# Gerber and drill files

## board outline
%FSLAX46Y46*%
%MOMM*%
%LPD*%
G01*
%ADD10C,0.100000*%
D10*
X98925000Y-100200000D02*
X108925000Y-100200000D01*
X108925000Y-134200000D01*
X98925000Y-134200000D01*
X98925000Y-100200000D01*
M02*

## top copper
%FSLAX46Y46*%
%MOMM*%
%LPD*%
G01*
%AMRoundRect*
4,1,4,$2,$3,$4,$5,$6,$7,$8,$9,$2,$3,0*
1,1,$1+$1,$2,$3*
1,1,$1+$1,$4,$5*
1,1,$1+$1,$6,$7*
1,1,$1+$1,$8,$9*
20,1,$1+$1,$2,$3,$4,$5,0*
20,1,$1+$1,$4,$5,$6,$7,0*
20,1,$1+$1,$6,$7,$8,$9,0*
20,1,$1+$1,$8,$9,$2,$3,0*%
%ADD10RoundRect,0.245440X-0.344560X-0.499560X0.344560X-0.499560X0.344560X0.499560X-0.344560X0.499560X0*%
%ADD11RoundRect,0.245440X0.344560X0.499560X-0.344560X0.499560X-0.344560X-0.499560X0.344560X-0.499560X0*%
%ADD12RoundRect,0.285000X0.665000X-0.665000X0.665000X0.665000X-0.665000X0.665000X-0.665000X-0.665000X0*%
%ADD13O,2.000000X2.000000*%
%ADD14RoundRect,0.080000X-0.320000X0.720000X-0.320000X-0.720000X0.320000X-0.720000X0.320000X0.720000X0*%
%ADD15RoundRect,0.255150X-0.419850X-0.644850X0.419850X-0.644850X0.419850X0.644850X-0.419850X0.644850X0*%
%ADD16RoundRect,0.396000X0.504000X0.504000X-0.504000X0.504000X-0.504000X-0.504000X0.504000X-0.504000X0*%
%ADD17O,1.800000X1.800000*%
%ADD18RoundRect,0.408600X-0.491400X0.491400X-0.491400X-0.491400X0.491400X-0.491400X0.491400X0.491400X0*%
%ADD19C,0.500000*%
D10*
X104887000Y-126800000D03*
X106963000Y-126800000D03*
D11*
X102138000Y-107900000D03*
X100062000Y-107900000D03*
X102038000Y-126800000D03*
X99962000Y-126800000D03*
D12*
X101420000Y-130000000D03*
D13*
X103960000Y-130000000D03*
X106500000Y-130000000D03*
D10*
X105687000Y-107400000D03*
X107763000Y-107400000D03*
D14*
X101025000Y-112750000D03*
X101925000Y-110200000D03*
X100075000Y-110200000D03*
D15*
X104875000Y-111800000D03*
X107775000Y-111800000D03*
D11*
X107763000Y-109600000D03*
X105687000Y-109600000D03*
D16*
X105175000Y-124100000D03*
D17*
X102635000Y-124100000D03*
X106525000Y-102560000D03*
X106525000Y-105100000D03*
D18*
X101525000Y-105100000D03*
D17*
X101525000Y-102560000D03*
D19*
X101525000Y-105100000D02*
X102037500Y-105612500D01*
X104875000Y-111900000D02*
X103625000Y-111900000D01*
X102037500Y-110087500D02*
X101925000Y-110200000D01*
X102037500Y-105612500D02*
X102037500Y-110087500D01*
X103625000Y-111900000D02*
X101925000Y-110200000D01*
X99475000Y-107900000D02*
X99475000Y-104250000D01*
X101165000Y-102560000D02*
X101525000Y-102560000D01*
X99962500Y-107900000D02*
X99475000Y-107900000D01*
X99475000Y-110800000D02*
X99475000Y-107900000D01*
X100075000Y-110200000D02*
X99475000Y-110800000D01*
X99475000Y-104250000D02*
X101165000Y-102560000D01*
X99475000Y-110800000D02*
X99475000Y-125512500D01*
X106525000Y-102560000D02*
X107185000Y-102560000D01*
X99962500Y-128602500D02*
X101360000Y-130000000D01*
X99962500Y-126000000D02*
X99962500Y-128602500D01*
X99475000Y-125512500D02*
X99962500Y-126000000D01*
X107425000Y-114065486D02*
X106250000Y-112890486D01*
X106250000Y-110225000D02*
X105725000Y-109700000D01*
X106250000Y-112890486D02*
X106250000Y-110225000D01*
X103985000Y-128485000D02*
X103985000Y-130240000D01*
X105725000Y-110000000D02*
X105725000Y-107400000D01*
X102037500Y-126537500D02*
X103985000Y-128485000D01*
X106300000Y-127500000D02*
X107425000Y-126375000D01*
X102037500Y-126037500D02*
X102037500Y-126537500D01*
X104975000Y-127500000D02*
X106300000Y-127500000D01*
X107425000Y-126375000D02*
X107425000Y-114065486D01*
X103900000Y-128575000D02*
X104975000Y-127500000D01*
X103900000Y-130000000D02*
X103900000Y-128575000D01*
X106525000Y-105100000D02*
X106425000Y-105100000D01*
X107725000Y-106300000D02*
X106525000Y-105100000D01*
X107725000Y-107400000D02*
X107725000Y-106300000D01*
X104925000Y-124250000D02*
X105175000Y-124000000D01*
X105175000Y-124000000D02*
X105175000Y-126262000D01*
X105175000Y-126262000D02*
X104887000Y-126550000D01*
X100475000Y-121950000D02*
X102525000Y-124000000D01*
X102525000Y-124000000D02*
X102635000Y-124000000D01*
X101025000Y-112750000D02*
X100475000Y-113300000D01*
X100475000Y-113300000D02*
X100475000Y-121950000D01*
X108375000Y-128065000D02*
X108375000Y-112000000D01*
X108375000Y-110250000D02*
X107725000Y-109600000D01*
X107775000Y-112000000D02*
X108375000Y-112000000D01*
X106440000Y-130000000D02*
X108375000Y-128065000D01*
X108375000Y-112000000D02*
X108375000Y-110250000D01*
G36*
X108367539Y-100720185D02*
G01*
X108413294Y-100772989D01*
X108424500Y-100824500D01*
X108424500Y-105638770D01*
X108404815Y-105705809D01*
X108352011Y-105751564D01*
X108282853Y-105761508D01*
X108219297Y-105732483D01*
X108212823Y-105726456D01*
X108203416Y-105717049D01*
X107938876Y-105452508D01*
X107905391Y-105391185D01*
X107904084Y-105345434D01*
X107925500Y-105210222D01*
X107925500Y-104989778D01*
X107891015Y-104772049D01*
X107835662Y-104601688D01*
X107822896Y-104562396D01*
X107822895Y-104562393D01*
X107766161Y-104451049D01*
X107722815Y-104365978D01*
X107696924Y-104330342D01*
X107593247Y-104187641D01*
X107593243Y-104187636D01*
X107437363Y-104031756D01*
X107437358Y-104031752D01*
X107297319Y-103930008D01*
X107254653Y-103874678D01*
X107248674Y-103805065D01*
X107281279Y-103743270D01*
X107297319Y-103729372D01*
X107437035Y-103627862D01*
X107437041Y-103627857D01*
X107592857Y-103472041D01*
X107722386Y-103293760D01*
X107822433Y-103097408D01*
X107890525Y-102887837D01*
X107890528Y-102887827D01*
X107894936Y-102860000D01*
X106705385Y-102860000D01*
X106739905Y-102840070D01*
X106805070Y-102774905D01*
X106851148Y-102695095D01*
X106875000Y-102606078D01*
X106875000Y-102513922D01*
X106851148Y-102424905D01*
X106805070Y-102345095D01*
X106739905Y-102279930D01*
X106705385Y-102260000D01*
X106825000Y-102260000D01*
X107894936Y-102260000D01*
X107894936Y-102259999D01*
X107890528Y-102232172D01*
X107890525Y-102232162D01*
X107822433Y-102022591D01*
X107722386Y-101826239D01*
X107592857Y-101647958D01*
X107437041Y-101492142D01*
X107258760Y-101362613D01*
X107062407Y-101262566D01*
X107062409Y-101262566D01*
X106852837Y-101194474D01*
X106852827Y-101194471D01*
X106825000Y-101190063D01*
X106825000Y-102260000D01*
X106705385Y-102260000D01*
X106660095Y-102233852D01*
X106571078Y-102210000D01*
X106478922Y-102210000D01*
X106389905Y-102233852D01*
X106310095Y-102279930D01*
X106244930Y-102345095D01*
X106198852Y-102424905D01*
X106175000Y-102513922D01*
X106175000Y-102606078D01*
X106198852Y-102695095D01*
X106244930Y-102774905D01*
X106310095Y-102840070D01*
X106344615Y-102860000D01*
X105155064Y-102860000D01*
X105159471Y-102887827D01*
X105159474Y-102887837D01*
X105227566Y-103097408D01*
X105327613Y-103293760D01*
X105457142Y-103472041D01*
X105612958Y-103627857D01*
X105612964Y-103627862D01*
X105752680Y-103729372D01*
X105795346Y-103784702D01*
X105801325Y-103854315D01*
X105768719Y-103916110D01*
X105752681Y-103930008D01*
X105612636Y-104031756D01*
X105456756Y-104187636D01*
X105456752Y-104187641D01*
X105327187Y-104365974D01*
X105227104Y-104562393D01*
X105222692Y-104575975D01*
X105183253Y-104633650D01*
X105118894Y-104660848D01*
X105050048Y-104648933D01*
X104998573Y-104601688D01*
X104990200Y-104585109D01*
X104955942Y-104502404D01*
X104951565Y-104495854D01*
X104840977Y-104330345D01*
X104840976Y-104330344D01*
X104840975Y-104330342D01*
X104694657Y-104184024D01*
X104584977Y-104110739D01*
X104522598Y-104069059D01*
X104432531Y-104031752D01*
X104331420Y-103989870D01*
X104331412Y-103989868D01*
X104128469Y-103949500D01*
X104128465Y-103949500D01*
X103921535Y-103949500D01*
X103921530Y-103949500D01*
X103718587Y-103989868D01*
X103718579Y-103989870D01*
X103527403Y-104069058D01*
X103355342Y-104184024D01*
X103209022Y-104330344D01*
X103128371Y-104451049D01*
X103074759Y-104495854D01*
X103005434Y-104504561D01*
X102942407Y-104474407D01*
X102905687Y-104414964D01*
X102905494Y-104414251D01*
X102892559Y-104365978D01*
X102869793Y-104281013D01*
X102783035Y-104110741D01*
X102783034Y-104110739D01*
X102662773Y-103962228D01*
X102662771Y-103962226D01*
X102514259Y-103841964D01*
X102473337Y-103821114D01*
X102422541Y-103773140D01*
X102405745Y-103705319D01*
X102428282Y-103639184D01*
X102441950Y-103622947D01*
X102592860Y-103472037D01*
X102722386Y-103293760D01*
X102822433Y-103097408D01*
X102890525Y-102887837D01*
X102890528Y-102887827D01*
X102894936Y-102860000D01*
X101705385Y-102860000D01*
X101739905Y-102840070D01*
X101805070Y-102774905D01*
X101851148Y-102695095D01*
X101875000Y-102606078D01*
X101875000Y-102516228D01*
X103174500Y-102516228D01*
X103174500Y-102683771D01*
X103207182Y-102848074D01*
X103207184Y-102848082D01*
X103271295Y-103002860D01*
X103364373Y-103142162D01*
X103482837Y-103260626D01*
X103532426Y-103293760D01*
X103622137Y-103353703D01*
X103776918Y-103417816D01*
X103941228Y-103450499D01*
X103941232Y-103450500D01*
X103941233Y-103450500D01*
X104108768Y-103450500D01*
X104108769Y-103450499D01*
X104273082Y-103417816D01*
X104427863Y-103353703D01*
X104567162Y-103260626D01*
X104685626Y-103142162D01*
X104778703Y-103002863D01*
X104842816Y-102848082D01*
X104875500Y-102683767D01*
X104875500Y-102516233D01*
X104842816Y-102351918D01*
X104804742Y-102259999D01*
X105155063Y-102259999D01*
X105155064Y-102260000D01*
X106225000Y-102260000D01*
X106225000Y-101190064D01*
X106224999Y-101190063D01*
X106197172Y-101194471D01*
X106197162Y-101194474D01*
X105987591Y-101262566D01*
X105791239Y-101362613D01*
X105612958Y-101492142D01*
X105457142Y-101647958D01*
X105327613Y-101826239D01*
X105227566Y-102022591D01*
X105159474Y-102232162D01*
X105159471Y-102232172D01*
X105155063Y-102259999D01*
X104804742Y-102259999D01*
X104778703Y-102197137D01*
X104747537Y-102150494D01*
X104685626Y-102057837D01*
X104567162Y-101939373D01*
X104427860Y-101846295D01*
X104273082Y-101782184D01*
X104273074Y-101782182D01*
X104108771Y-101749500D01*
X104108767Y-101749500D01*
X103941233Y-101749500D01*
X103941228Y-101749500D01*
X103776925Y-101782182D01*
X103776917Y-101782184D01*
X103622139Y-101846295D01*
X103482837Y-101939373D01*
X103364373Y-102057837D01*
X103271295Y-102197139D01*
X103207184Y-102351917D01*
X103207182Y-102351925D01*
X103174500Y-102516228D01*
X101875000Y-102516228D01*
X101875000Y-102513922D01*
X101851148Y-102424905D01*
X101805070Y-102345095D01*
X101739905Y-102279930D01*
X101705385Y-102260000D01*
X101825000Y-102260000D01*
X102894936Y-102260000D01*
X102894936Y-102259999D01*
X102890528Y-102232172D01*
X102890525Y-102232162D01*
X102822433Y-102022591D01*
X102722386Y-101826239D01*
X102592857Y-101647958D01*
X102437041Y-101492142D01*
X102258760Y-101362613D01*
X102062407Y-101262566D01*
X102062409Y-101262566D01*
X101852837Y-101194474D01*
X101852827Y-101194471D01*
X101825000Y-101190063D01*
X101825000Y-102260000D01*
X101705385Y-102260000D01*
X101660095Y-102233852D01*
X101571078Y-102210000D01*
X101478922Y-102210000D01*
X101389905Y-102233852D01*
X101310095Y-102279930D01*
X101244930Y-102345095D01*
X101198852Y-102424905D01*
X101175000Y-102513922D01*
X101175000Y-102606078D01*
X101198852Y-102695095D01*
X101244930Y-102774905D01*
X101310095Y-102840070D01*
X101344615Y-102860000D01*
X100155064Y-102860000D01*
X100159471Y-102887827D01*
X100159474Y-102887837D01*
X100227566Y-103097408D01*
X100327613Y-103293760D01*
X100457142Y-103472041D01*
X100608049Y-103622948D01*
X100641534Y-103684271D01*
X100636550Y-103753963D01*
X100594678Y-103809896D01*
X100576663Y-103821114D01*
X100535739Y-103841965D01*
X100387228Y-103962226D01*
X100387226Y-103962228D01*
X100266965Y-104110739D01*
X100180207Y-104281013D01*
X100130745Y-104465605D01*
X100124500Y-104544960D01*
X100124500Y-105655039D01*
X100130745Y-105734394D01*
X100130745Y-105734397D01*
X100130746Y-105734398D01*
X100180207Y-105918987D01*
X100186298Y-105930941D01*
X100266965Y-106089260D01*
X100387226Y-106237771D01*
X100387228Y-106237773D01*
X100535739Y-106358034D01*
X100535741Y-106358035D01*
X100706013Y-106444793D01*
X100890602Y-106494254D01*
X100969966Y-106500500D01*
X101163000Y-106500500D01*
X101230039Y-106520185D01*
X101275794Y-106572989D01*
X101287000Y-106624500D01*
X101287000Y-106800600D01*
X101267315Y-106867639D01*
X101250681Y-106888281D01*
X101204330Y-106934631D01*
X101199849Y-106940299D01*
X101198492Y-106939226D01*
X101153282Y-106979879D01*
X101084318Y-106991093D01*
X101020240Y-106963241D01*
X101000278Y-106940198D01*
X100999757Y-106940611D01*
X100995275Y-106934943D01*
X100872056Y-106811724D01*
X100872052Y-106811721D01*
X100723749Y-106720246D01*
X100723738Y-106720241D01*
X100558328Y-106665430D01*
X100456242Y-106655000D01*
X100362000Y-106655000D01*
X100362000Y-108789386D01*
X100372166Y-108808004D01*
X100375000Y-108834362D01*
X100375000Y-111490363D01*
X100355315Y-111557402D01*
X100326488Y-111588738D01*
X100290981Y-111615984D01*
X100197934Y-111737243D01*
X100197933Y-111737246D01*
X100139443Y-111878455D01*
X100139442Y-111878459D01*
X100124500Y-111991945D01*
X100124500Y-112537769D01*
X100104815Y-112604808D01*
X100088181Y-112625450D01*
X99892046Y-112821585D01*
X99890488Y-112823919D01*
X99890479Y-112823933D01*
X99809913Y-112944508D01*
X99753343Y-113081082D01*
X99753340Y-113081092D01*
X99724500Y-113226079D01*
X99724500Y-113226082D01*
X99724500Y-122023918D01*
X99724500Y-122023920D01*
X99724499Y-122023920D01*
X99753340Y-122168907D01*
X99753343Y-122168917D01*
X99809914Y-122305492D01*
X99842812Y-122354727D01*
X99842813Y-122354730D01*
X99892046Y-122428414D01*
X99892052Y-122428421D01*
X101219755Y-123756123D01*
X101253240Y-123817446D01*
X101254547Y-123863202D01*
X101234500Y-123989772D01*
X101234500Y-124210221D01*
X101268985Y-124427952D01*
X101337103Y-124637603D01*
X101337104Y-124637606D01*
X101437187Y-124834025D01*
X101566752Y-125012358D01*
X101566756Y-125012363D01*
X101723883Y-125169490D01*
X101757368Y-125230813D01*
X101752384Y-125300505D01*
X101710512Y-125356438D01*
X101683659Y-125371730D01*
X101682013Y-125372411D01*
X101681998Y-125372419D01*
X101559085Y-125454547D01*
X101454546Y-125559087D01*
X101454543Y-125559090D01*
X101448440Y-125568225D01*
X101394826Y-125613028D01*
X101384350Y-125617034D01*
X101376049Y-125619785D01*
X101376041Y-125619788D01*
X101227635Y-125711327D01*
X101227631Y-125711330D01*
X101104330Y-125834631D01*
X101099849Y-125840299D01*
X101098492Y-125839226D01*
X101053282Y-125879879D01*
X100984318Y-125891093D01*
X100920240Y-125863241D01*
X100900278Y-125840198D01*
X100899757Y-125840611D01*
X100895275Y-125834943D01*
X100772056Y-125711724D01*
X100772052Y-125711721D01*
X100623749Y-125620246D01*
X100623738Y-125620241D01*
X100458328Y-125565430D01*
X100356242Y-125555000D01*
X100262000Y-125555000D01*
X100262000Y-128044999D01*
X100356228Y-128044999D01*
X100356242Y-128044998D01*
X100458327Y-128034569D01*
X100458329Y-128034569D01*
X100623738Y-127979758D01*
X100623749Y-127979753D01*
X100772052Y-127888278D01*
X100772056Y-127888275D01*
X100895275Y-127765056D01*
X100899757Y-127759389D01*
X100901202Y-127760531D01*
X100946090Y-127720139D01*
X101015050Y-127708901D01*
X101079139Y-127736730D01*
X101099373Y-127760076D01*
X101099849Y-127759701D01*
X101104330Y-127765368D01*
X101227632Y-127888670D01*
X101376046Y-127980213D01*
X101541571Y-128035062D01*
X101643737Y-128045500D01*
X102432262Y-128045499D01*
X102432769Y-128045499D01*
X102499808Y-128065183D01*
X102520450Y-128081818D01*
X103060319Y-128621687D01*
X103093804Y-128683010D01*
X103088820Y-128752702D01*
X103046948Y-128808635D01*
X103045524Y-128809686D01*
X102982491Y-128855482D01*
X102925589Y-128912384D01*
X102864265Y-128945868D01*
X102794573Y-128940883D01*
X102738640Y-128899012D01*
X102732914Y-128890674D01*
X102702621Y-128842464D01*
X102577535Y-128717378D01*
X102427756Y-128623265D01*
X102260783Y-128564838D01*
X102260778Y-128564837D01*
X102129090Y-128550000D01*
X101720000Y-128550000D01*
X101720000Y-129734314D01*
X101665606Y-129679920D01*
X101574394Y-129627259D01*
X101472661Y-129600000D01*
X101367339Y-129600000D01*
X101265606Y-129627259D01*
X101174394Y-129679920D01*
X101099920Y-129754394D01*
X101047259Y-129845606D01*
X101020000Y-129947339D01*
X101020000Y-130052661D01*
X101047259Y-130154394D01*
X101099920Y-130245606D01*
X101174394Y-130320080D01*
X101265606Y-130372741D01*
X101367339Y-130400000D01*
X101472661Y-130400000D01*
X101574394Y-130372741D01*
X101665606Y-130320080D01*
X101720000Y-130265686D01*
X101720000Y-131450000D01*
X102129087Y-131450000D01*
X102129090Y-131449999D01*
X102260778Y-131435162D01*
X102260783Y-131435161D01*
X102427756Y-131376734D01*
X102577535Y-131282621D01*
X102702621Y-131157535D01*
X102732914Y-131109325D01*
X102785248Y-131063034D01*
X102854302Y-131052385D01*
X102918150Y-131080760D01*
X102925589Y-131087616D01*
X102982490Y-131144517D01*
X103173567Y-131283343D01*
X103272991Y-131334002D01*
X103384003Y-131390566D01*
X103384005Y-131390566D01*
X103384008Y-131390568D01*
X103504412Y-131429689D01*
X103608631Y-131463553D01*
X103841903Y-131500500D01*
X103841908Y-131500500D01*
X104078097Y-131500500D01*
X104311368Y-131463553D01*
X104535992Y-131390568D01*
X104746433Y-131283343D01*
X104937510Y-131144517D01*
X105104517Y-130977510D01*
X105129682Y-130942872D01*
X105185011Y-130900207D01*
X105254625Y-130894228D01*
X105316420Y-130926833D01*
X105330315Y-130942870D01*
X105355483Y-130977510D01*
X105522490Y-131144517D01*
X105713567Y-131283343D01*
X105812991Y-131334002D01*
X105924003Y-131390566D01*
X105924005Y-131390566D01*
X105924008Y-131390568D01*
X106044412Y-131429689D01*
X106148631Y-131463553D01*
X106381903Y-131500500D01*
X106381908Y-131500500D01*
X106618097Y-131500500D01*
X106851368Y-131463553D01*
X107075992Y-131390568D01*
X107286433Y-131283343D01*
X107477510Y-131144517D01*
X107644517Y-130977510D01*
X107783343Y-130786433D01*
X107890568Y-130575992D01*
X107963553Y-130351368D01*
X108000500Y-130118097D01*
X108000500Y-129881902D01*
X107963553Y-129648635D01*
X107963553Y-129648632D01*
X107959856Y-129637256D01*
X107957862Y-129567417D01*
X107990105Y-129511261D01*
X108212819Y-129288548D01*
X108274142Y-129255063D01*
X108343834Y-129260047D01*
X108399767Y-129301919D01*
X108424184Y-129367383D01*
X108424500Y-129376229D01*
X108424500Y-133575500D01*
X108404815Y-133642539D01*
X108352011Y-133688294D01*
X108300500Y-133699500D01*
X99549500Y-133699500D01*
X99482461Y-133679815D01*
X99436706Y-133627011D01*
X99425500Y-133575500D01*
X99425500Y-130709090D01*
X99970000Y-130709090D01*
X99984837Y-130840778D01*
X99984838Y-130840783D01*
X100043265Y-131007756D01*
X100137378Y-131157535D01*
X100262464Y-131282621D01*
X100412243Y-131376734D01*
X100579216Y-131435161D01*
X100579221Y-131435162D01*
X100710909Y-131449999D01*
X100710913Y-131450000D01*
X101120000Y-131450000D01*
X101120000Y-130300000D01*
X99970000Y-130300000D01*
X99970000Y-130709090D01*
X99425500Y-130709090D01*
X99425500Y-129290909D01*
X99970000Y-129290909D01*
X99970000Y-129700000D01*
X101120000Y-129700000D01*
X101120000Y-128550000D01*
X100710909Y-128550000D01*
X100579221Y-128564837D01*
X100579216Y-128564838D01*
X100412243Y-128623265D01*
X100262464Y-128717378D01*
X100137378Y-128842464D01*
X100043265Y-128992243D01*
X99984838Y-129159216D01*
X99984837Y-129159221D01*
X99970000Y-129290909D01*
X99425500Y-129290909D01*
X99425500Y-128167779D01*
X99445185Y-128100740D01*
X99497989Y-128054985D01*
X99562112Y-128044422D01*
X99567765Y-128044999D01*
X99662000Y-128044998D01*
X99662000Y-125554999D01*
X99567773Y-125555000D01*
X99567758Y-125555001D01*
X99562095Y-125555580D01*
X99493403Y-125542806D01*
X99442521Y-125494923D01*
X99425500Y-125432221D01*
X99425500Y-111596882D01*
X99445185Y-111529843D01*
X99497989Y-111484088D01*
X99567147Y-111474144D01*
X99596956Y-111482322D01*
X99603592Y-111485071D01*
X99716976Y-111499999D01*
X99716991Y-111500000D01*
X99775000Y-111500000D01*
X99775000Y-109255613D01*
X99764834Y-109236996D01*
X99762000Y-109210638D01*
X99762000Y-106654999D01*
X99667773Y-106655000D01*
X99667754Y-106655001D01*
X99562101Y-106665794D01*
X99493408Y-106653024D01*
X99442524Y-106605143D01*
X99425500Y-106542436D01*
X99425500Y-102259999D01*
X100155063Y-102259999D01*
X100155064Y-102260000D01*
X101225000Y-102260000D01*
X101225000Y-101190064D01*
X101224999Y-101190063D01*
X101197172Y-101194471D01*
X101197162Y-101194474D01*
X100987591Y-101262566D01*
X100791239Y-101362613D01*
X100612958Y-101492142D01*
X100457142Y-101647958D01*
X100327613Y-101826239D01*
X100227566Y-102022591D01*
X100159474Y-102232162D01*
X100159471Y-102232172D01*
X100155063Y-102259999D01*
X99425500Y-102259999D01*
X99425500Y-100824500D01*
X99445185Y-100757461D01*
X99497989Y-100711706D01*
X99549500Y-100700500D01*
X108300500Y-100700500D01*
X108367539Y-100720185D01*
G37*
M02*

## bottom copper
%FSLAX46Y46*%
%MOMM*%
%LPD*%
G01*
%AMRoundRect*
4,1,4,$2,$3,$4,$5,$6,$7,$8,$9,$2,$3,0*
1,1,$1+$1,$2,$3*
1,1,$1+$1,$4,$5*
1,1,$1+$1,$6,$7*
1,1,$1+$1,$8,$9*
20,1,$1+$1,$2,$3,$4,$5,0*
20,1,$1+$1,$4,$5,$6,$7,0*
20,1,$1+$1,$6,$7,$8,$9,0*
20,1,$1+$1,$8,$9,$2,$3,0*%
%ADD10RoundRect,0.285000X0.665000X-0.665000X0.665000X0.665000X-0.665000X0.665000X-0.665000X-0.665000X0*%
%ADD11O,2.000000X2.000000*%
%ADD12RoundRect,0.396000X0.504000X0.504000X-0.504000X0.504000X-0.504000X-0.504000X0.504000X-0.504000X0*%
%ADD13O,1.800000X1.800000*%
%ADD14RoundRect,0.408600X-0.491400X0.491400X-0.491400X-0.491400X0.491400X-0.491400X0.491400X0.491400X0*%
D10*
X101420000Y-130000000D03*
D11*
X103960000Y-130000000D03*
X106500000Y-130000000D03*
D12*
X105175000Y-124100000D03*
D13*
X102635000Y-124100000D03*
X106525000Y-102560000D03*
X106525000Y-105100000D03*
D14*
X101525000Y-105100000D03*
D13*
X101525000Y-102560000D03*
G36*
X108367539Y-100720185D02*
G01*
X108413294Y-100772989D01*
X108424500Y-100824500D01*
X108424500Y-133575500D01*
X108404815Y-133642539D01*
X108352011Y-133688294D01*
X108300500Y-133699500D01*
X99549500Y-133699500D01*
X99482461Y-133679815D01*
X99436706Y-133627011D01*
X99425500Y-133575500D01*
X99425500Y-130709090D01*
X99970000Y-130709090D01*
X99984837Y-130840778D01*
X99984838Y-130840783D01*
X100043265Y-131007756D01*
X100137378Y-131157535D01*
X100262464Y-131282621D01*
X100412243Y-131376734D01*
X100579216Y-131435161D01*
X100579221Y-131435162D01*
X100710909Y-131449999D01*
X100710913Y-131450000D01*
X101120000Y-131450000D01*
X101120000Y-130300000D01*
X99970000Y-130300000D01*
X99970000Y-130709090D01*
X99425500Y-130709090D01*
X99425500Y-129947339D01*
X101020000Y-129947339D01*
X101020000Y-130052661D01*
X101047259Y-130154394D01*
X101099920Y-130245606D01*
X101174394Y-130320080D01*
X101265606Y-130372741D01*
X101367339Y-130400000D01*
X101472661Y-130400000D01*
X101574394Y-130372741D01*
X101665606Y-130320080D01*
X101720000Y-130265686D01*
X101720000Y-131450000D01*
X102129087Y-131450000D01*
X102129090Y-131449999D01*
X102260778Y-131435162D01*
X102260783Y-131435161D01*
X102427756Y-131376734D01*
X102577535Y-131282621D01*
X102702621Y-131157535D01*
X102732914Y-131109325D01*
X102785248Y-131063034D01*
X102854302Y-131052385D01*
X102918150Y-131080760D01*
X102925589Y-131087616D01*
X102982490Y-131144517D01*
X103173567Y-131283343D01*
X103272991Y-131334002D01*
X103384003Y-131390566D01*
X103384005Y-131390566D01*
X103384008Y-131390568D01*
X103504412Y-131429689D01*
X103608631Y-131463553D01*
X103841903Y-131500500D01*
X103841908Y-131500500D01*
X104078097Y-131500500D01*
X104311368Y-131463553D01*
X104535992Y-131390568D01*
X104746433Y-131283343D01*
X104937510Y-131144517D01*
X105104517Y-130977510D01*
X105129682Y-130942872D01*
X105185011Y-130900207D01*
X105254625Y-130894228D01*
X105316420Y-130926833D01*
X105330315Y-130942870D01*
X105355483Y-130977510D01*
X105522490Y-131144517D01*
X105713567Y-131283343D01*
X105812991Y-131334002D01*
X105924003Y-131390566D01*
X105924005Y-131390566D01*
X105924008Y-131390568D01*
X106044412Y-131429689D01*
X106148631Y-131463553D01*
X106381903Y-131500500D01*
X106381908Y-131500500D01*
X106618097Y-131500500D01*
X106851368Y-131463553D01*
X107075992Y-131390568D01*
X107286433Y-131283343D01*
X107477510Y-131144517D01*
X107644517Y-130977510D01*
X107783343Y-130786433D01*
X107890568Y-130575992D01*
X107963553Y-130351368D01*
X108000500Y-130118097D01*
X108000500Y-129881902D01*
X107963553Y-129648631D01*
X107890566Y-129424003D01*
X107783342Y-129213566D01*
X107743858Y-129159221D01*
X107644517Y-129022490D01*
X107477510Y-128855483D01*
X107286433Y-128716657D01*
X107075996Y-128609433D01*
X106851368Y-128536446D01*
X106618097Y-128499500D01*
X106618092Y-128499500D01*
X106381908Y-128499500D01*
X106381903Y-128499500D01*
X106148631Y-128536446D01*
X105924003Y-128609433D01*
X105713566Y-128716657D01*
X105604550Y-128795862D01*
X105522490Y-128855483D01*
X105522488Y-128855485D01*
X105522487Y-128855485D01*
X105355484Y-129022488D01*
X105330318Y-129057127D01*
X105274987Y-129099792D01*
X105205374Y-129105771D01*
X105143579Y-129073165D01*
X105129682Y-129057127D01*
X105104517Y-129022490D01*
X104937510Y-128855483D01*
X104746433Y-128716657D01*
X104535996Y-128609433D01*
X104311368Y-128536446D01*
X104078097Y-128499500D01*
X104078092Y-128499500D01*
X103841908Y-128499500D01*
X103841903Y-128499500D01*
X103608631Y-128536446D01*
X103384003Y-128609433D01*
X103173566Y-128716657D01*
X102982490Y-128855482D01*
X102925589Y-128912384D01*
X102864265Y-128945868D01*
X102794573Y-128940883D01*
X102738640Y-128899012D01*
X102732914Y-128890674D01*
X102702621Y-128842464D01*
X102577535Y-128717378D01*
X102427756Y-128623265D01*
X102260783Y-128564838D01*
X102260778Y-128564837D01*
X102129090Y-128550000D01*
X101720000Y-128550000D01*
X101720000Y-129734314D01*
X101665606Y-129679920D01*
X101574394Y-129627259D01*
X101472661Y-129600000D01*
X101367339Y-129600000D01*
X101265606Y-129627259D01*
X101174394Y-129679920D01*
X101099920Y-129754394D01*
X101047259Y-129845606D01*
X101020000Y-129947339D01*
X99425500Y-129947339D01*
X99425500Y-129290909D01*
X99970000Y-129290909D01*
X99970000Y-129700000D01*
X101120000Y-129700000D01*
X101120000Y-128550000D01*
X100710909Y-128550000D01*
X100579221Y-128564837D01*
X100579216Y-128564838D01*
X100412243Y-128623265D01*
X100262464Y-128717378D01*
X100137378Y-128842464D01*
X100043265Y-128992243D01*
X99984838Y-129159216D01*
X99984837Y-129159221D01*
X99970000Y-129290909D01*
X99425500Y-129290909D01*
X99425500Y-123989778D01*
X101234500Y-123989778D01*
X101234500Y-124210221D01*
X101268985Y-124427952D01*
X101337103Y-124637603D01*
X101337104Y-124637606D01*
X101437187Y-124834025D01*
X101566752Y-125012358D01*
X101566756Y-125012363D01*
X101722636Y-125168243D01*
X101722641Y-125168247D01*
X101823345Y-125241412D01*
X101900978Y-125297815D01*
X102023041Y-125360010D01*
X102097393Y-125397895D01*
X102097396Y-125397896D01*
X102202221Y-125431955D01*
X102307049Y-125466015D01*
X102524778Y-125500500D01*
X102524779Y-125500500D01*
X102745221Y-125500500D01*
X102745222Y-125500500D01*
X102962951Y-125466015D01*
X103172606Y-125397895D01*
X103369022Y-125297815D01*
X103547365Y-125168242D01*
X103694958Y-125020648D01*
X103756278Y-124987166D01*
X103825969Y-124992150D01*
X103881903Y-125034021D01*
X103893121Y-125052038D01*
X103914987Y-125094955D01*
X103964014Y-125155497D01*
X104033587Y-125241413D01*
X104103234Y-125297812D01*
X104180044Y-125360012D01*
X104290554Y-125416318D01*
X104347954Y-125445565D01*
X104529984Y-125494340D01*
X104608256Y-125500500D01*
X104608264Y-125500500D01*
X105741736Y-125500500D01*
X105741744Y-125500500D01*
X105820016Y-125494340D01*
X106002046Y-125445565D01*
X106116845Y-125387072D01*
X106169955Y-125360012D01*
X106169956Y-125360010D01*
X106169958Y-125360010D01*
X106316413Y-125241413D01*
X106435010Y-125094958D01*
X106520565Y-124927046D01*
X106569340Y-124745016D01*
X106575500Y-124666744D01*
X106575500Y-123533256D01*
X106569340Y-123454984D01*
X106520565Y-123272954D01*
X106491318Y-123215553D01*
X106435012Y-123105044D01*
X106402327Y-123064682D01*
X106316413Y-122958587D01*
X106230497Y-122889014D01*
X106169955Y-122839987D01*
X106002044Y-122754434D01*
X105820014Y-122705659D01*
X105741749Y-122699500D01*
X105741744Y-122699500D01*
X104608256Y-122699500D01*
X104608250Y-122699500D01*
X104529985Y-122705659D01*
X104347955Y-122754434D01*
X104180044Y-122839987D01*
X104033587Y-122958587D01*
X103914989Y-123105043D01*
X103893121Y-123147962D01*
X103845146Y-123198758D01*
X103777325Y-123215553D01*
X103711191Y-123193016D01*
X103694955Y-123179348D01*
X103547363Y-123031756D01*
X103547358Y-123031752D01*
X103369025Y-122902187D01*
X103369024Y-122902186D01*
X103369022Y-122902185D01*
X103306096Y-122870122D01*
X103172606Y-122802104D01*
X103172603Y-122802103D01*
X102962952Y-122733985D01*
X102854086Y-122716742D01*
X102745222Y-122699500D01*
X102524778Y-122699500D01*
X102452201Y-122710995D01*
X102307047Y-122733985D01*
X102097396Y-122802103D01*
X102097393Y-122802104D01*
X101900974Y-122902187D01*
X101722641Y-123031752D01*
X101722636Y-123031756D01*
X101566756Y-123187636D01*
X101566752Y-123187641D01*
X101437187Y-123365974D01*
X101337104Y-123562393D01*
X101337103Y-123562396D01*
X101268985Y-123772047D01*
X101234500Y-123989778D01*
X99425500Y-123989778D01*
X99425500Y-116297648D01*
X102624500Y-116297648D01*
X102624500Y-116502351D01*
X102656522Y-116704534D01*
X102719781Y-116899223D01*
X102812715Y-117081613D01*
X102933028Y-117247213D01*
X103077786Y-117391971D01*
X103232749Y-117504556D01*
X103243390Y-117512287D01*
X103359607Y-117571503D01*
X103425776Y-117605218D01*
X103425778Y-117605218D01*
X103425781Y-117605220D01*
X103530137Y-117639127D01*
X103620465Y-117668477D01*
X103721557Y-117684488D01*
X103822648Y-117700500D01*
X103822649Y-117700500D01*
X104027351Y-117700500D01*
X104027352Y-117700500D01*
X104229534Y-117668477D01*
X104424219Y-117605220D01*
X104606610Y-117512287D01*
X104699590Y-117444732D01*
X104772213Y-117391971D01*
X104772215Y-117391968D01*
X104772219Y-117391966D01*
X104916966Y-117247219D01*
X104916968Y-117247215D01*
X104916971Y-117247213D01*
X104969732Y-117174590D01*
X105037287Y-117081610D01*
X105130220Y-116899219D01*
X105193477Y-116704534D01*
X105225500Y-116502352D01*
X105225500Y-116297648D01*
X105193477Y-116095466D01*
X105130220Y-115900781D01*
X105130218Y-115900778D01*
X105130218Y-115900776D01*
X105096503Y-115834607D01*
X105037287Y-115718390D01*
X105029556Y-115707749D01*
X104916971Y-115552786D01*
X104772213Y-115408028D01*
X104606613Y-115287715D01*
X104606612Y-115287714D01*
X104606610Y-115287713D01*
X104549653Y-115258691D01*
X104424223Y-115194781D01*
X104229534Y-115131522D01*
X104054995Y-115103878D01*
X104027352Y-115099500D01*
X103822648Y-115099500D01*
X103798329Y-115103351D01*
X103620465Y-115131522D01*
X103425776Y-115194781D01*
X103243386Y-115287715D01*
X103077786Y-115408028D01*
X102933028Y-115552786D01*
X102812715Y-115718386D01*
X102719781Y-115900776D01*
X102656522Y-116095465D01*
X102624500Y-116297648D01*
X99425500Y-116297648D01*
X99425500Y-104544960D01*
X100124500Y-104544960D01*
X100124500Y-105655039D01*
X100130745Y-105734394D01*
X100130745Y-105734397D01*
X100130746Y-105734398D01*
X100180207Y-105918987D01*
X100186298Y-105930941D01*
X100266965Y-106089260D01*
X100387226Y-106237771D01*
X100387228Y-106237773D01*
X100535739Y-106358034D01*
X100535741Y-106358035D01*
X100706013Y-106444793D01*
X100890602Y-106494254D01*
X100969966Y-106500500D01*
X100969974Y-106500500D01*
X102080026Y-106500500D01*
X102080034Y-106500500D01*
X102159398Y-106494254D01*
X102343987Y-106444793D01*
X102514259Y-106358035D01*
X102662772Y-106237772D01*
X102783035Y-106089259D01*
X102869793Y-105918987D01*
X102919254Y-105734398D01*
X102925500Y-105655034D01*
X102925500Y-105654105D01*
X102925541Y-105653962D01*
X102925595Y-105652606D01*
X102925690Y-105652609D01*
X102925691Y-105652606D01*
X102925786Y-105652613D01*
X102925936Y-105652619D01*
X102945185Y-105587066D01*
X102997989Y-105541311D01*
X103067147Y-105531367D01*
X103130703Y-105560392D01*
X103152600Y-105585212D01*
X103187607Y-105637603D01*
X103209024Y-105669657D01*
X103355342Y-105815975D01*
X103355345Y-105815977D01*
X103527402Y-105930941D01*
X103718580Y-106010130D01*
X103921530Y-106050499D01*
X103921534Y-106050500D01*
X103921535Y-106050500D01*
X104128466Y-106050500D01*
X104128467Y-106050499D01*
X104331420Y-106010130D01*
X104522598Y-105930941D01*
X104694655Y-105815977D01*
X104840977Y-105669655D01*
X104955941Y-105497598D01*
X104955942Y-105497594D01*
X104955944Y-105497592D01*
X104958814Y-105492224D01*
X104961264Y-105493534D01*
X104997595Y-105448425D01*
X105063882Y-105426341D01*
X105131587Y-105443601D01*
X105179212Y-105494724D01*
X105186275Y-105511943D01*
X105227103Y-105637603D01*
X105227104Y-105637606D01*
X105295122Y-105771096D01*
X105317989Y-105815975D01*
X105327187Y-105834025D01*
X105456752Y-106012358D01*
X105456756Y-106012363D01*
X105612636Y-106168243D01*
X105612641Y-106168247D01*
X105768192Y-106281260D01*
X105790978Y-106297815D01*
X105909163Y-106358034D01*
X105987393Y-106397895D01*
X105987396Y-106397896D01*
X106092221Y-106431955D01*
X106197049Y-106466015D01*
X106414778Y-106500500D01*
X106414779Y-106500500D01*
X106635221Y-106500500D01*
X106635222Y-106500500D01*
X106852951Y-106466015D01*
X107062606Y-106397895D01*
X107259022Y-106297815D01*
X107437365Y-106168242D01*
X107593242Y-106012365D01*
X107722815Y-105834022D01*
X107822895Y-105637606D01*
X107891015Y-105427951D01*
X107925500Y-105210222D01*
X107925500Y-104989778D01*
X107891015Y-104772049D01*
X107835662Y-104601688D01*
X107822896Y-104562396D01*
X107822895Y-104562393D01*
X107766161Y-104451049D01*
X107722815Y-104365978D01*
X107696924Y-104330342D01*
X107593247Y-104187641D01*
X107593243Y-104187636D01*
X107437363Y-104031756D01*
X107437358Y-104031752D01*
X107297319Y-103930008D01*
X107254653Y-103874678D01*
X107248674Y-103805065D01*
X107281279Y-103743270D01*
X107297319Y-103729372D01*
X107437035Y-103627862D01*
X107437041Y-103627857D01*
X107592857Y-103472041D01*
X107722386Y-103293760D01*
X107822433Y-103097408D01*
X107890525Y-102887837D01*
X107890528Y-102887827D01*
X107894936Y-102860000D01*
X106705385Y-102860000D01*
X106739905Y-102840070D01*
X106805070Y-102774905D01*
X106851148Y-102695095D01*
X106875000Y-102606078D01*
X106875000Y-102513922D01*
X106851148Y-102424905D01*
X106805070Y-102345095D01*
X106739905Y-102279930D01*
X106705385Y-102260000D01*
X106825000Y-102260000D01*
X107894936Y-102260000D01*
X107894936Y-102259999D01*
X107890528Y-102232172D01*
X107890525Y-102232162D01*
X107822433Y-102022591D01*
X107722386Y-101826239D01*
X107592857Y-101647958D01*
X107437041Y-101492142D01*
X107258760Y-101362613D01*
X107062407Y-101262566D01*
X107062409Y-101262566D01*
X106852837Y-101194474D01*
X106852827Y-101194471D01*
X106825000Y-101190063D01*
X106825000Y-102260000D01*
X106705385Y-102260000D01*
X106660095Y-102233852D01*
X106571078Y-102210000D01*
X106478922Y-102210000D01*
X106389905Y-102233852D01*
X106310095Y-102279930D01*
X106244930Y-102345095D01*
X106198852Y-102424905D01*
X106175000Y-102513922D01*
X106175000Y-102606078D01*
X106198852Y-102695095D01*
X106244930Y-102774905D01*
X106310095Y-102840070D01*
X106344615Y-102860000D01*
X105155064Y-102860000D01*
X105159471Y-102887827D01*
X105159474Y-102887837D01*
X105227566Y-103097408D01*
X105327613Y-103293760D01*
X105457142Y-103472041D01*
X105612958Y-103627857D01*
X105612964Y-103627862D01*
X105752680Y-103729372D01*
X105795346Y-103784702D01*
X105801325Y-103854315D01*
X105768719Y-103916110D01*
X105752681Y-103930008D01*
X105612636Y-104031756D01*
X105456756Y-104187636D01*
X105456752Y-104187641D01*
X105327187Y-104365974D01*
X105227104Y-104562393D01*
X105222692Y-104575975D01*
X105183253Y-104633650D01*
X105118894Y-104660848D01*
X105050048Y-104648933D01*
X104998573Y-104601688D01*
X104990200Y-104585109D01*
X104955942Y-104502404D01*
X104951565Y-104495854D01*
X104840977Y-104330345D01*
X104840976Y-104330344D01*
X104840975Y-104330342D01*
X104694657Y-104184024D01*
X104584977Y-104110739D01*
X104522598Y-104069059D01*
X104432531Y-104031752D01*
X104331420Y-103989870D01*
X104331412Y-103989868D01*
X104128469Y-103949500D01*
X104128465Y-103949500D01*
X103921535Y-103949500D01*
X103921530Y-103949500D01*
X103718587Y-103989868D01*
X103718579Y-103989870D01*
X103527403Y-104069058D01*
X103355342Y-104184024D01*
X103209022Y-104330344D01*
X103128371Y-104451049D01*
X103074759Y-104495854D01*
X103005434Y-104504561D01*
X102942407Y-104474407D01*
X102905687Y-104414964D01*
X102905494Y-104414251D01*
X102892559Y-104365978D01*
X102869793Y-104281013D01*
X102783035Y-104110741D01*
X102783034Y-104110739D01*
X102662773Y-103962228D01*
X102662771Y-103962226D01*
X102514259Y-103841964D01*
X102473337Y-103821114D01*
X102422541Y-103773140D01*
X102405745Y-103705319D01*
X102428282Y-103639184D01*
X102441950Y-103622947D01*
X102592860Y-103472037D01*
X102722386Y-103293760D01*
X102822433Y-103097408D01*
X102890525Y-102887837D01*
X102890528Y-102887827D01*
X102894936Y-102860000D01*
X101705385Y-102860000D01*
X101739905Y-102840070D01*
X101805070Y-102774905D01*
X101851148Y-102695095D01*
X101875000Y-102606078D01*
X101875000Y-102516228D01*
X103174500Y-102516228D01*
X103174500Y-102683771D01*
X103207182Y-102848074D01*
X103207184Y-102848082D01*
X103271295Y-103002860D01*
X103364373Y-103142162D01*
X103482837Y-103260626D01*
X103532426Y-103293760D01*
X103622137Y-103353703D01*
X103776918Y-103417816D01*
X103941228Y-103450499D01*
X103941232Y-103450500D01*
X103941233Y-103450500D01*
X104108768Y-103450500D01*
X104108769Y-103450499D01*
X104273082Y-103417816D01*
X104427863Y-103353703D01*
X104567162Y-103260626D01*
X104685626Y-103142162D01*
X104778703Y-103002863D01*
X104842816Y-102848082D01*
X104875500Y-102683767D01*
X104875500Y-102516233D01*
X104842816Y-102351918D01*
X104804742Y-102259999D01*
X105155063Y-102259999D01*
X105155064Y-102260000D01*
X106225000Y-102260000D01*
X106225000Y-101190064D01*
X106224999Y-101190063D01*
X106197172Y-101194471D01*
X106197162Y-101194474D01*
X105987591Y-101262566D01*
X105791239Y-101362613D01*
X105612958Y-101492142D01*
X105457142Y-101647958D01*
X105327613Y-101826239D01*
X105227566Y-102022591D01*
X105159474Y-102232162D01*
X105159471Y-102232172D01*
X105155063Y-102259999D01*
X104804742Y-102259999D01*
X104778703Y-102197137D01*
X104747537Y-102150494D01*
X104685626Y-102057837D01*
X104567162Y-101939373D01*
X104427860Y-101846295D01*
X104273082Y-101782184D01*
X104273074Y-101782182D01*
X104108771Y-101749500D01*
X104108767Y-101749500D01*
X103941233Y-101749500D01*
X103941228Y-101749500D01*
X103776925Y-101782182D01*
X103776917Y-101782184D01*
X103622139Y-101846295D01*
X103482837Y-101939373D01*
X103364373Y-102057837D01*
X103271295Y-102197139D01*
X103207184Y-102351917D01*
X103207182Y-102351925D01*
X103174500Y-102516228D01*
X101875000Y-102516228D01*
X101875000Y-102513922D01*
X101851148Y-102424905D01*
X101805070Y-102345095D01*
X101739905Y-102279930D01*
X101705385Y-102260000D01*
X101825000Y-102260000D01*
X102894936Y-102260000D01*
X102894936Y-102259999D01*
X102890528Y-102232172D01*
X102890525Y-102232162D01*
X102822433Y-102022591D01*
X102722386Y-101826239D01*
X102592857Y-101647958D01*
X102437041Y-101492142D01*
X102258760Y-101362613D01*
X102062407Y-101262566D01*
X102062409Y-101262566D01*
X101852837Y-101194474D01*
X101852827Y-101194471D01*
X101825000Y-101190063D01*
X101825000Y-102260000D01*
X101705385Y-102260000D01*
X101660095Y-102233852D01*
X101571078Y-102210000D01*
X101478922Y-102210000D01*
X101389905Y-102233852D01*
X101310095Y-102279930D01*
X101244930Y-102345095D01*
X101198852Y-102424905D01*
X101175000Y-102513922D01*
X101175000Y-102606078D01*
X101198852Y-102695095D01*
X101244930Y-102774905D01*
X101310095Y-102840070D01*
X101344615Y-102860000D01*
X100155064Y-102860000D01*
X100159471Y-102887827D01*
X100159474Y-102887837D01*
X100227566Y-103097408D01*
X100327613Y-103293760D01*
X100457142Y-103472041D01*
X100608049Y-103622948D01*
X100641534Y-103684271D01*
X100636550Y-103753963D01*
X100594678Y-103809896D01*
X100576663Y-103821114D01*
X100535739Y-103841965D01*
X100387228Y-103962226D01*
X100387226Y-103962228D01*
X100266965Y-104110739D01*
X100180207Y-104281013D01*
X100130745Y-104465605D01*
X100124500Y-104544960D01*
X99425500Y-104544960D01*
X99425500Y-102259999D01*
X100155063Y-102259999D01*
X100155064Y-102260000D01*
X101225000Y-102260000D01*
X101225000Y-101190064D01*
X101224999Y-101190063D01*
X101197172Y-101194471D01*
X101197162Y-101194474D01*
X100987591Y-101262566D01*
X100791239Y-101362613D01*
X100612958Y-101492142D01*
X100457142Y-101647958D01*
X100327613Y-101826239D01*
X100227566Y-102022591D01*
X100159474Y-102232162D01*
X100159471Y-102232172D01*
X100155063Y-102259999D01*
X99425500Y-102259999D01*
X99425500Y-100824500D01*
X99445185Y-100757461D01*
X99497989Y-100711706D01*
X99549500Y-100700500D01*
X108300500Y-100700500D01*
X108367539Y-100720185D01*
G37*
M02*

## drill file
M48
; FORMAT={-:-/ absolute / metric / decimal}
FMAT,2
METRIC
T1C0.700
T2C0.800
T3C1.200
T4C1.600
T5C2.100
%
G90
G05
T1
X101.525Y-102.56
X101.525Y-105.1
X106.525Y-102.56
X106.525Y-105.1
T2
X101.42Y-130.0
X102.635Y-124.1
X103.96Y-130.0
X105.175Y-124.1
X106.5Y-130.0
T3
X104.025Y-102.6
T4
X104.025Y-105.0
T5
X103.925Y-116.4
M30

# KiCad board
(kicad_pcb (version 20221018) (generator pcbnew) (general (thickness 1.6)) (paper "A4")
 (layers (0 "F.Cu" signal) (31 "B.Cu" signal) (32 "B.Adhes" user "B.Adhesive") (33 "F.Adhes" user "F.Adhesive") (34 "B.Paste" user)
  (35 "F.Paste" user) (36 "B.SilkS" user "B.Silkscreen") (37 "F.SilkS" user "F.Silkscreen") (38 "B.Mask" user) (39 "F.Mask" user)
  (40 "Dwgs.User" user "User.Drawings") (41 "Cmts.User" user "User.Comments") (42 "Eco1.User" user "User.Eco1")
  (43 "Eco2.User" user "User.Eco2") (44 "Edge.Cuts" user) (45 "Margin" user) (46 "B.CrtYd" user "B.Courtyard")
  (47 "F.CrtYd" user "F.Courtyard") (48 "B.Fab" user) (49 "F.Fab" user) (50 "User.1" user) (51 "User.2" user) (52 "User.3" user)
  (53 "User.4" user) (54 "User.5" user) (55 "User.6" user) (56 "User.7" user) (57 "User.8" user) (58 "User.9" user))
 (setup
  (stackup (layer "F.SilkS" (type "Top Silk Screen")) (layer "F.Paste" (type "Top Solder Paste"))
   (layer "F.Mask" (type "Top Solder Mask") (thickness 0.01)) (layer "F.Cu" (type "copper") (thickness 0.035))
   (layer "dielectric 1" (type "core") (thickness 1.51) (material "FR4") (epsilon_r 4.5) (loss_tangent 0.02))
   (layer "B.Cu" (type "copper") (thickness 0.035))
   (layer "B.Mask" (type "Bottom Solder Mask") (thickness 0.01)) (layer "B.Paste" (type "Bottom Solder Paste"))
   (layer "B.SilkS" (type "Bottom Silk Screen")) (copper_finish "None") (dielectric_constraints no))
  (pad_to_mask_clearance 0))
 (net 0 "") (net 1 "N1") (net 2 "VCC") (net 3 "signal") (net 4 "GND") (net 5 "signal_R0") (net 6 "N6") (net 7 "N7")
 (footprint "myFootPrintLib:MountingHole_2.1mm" (layer "F.Cu") (at 103.925 116.4 180)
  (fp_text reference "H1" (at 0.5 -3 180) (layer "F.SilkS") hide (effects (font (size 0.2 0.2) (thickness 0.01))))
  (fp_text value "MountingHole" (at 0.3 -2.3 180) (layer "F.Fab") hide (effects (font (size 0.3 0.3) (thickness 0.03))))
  (pad "" np_thru_hole circle (at 0 0 180) (size 2.1 2.1) (drill 2.1) (layers "F&B.Cu" "*.Mask")))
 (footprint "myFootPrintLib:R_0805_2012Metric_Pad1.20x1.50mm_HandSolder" (layer "F.Cu") (at 105.925 126.8)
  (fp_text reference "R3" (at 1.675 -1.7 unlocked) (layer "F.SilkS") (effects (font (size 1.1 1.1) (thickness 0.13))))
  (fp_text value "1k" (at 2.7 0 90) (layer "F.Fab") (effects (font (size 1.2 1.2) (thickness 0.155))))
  (pad "1" smd roundrect (at -1.038 0) (size 1.18 1.49) (layers "F.Cu" "F.Paste" "F.Mask") (roundrect_rratio 0.208) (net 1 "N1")
   (solder_mask_margin 0.05))
  (pad "2" smd roundrect (at 1.038 0) (size 1.18 1.49) (layers "F.Cu" "F.Paste" "F.Mask") (roundrect_rratio 0.208) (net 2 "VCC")
   (solder_mask_margin 0.05)))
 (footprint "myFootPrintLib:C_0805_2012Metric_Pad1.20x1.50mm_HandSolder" (layer "F.Cu") (at 101.1 107.9 180)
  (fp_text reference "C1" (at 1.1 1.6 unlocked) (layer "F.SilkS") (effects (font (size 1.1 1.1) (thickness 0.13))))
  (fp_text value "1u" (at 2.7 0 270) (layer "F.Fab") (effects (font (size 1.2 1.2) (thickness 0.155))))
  (pad "1" smd roundrect (at -1.038 0 180) (size 1.18 1.49) (layers "F.Cu" "F.Paste" "F.Mask") (roundrect_rratio 0.208) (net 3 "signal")
   (solder_mask_margin 0.05))
  (pad "2" smd roundrect (at 1.038 0 180) (size 1.18 1.49) (layers "F.Cu" "F.Paste" "F.Mask") (roundrect_rratio 0.208) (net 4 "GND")
   (solder_mask_margin 0.05)))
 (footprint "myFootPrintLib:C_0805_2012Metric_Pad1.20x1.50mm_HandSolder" (layer "F.Cu") (at 101 126.8 180)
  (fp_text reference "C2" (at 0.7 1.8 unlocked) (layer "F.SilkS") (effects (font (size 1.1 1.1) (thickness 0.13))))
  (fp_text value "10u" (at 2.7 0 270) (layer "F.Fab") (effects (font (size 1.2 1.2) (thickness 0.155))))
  (pad "1" smd roundrect (at -1.038 0 180) (size 1.18 1.49) (layers "F.Cu" "F.Paste" "F.Mask") (roundrect_rratio 0.208) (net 2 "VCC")
   (solder_mask_margin 0.05))
  (pad "2" smd roundrect (at 1.038 0 180) (size 1.18 1.49) (layers "F.Cu" "F.Paste" "F.Mask") (roundrect_rratio 0.208) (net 4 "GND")
   (solder_mask_margin 0.05)))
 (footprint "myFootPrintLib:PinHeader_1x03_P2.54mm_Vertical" (layer "F.Cu") (at 101.42 130 90)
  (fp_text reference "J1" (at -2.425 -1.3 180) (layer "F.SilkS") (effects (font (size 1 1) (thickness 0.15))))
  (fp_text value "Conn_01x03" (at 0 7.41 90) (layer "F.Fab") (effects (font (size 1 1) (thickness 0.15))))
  (pad "1" thru_hole roundrect (at 0 0 90) (size 1.9 1.9) (drill 0.8) (layers "*.Cu" "*.Mask") (roundrect_rratio 0.15) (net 4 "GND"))
  (pad "2" thru_hole oval (at 0 2.54 90) (size 2 2) (drill 0.8) (layers "*.Cu" "*.Mask") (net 2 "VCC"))
  (pad "3" thru_hole oval (at 0 5.08 90) (size 2 2) (drill 0.8) (layers "*.Cu" "*.Mask") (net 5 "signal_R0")))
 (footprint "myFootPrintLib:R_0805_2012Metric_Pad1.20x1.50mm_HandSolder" (layer "F.Cu") (at 106.725 107.4)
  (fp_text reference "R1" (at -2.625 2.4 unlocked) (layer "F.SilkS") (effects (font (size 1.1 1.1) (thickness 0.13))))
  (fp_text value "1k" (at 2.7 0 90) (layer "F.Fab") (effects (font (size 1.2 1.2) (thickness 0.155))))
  (pad "1" smd roundrect (at -1.038 0) (size 1.18 1.49) (layers "F.Cu" "F.Paste" "F.Mask") (roundrect_rratio 0.208) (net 2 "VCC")
   (solder_mask_margin 0.05))
  (pad "2" smd roundrect (at 1.038 0) (size 1.18 1.49) (layers "F.Cu" "F.Paste" "F.Mask") (roundrect_rratio 0.208) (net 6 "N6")
   (solder_mask_margin 0.05)))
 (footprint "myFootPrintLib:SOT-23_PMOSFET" (layer "F.Cu") (at 101.025 111.45 -90)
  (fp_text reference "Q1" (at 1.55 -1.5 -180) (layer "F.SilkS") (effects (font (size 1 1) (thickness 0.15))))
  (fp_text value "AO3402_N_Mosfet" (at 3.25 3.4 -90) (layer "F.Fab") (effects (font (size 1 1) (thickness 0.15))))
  (pad "D" smd roundrect (at 1.3 0 270) (size 1.6 0.8) (layers "F.Cu" "F.Paste" "F.Mask") (roundrect_rratio 0.1) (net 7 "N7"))
  (pad "G" smd roundrect (at -1.25 -0.9 270) (size 1.6 0.8) (layers "F.Cu" "F.Paste" "F.Mask") (roundrect_rratio 0.1) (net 3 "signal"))
  (pad "S" smd roundrect (at -1.25 0.95 270) (size 1.6 0.8) (layers "F.Cu" "F.Paste" "F.Mask") (roundrect_rratio 0.1) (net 4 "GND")))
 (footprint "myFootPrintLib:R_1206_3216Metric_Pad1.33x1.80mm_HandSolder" (layer "F.Cu") (at 106.325 111.8)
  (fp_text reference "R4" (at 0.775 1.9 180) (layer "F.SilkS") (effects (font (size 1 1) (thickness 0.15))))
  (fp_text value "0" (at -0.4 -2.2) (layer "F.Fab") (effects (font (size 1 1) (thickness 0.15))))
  (pad "1" smd roundrect (at -1.45 0) (size 1.35 1.8) (layers "F.Cu" "F.Paste" "F.Mask") (roundrect_rratio 0.189) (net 3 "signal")
   (solder_mask_margin 0.05))
  (pad "2" smd roundrect (at 1.45 0) (size 1.35 1.8) (layers "F.Cu" "F.Paste" "F.Mask") (roundrect_rratio 0.189) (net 5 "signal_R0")
   (solder_mask_margin 0.05)))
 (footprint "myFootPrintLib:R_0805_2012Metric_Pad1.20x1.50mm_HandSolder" (layer "F.Cu") (at 106.725 109.6 180)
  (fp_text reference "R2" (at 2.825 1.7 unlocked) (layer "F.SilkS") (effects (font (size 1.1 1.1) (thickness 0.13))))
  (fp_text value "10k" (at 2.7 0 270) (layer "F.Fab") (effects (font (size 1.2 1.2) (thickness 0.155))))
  (pad "1" smd roundrect (at -1.038 0 180) (size 1.18 1.49) (layers "F.Cu" "F.Paste" "F.Mask") (roundrect_rratio 0.208) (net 5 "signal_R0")
   (solder_mask_margin 0.05))
  (pad "2" smd roundrect (at 1.038 0 180) (size 1.18 1.49) (layers "F.Cu" "F.Paste" "F.Mask") (roundrect_rratio 0.208) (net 2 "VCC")
   (solder_mask_margin 0.05)))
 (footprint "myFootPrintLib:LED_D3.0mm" (layer "B.Cu") (at 105.175 124.1 180)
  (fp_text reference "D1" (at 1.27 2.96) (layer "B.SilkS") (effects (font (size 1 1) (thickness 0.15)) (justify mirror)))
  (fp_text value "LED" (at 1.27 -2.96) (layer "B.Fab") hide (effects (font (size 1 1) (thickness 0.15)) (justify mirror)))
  (pad "A" thru_hole roundrect (at 0 0 180) (size 1.8 1.8) (drill 0.8) (layers "*.Cu" "*.Mask") (roundrect_rratio 0.22) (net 1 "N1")
   (zone_connect 2))
  (pad "K" thru_hole oval (at 2.54 0 180) (size 1.8 1.8) (drill 0.8) (layers "*.Cu" "*.Mask") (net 7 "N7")))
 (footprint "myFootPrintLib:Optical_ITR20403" (layer "B.Cu") (at 100.425 106.1)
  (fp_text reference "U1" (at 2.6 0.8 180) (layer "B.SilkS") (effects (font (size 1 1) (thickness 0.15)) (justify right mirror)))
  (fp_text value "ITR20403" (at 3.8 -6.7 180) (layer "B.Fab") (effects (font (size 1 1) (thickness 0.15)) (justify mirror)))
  (pad "" np_thru_hole circle (at 3.6 -3.5 270) (size 1.2 1.2) (drill 1.2) (layers "F&B.Cu" "*.Mask"))
  (pad "" np_thru_hole circle (at 3.6 -1.1 270) (size 1.6 1.6) (drill 1.6) (layers "F&B.Cu" "*.Mask"))
  (pad "1" thru_hole oval (at 6.1 -3.54 270) (size 1.8 1.8) (drill 0.7) (layers "*.Cu" "*.Mask") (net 4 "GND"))
  (pad "2" thru_hole oval (at 6.1 -1 270) (size 1.8 1.8) (drill 0.7) (layers "*.Cu" "*.Mask") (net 6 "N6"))
  (pad "3" thru_hole roundrect (at 1.1 -1 270) (size 1.8 1.8) (drill 0.7) (layers "*.Cu" "*.Mask") (roundrect_rratio 0.227) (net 3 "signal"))
  (pad "4" thru_hole oval (at 1.1 -3.54 270) (size 1.8 1.8) (drill 0.7) (layers "*.Cu" "*.Mask") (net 4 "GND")))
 (gr_rect (start 98.925 100.2) (end 108.925 134.2) (stroke (width 0.1) (type default)) (fill none) (layer "Edge.Cuts"))
 (segment (start 101.525 105.1) (end 102.0375 105.6125) (width 0.5) (layer "F.Cu") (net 3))
 (segment (start 104.875 111.9) (end 103.625 111.9) (width 0.5) (layer "F.Cu") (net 3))
 (segment (start 102.0375 110.0875) (end 101.925 110.2) (width 0.5) (layer "F.Cu") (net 3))
 (segment (start 102.0375 105.6125) (end 102.0375 110.0875) (width 0.5) (layer "F.Cu") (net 3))
 (segment (start 103.625 111.9) (end 101.925 110.2) (width 0.5) (layer "F.Cu") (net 3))
 (segment (start 99.475 107.9) (end 99.475 104.25) (width 0.5) (layer "F.Cu") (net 4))
 (segment (start 101.165 102.56) (end 101.525 102.56) (width 0.5) (layer "F.Cu") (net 4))
 (segment (start 99.9625 107.9) (end 99.475 107.9) (width 0.5) (layer "F.Cu") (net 4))
 (segment (start 99.475 110.8) (end 99.475 107.9) (width 0.5) (layer "F.Cu") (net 4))
 (segment (start 100.075 110.2) (end 99.475 110.8) (width 0.5) (layer "F.Cu") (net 4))
 (segment (start 99.475 104.25) (end 101.165 102.56) (width 0.5) (layer "F.Cu") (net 4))
 (segment (start 99.475 110.8) (end 99.475 125.5125) (width 0.5) (layer "F.Cu") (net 4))
 (segment (start 106.525 102.56) (end 107.185 102.56) (width 0.5) (layer "F.Cu") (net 4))
 (segment (start 99.9625 128.6025) (end 101.36 130) (width 0.5) (layer "F.Cu") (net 4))
 (segment (start 99.9625 126) (end 99.9625 128.6025) (width 0.5) (layer "F.Cu") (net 4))
 (segment (start 99.475 125.5125) (end 99.9625 126) (width 0.5) (layer "F.Cu") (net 4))
 (segment (start 107.425 114.065486) (end 106.25 112.890486) (width 0.5) (layer "F.Cu") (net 2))
 (segment (start 106.25 110.225) (end 105.725 109.7) (width 0.5) (layer "F.Cu") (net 2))
 (segment (start 106.25 112.890486) (end 106.25 110.225) (width 0.5) (layer "F.Cu") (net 2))
 (segment (start 103.985 128.485) (end 103.985 130.24) (width 0.5) (layer "F.Cu") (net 2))
 (segment (start 105.725 110) (end 105.725 107.4) (width 0.5) (layer "F.Cu") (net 2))
 (segment (start 102.0375 126.5375) (end 103.985 128.485) (width 0.5) (layer "F.Cu") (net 2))
 (segment (start 106.3 127.5) (end 107.425 126.375) (width 0.5) (layer "F.Cu") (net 2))
 (segment (start 102.0375 126.0375) (end 102.0375 126.5375) (width 0.5) (layer "F.Cu") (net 2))
 (segment (start 104.975 127.5) (end 106.3 127.5) (width 0.5) (layer "F.Cu") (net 2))
 (segment (start 107.425 126.375) (end 107.425 114.065486) (width 0.5) (layer "F.Cu") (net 2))
 (segment (start 103.9 128.575) (end 104.975 127.5) (width 0.5) (layer "F.Cu") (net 2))
 (segment (start 103.9 130) (end 103.9 128.575) (width 0.5) (layer "F.Cu") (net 2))
 (segment (start 106.525 105.1) (end 106.425 105.1) (width 0.5) (layer "F.Cu") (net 6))
 (segment (start 107.725 106.3) (end 106.525 105.1) (width 0.5) (layer "F.Cu") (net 6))
 (segment (start 107.725 107.4) (end 107.725 106.3) (width 0.5) (layer "F.Cu") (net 6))
 (segment (start 104.925 124.25) (end 105.175 124) (width 0.5) (layer "F.Cu") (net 1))
 (segment (start 105.175 124) (end 105.175 126.262) (width 0.5) (layer "F.Cu") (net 1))
 (segment (start 105.175 126.262) (end 104.887 126.55) (width 0.5) (layer "F.Cu") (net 1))
 (segment (start 100.475 121.95) (end 102.525 124) (width 0.5) (layer "F.Cu") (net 7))
 (segment (start 102.525 124) (end 102.635 124) (width 0.5) (layer "F.Cu") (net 7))
 (segment (start 101.025 112.75) (end 100.475 113.3) (width 0.5) (layer "F.Cu") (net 7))
 (segment (start 100.475 113.3) (end 100.475 121.95) (width 0.5) (layer "F.Cu") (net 7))
 (segment (start 108.375 128.065) (end 108.375 112) (width 0.5) (layer "F.Cu") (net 5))
 (segment (start 108.375 110.25) (end 107.725 109.6) (width 0.5) (layer "F.Cu") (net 5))
 (segment (start 107.775 112) (end 108.375 112) (width 0.5) (layer "F.Cu") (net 5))
 (segment (start 106.44 130) (end 108.375 128.065) (width 0.5) (layer "F.Cu") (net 5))
 (segment (start 108.375 112) (end 108.375 110.25) (width 0.5) (layer "F.Cu") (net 5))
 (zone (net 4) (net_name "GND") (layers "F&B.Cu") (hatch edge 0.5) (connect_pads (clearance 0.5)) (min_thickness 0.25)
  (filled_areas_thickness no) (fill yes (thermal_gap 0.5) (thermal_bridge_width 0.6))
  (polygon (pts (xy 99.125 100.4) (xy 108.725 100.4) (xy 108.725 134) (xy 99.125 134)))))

